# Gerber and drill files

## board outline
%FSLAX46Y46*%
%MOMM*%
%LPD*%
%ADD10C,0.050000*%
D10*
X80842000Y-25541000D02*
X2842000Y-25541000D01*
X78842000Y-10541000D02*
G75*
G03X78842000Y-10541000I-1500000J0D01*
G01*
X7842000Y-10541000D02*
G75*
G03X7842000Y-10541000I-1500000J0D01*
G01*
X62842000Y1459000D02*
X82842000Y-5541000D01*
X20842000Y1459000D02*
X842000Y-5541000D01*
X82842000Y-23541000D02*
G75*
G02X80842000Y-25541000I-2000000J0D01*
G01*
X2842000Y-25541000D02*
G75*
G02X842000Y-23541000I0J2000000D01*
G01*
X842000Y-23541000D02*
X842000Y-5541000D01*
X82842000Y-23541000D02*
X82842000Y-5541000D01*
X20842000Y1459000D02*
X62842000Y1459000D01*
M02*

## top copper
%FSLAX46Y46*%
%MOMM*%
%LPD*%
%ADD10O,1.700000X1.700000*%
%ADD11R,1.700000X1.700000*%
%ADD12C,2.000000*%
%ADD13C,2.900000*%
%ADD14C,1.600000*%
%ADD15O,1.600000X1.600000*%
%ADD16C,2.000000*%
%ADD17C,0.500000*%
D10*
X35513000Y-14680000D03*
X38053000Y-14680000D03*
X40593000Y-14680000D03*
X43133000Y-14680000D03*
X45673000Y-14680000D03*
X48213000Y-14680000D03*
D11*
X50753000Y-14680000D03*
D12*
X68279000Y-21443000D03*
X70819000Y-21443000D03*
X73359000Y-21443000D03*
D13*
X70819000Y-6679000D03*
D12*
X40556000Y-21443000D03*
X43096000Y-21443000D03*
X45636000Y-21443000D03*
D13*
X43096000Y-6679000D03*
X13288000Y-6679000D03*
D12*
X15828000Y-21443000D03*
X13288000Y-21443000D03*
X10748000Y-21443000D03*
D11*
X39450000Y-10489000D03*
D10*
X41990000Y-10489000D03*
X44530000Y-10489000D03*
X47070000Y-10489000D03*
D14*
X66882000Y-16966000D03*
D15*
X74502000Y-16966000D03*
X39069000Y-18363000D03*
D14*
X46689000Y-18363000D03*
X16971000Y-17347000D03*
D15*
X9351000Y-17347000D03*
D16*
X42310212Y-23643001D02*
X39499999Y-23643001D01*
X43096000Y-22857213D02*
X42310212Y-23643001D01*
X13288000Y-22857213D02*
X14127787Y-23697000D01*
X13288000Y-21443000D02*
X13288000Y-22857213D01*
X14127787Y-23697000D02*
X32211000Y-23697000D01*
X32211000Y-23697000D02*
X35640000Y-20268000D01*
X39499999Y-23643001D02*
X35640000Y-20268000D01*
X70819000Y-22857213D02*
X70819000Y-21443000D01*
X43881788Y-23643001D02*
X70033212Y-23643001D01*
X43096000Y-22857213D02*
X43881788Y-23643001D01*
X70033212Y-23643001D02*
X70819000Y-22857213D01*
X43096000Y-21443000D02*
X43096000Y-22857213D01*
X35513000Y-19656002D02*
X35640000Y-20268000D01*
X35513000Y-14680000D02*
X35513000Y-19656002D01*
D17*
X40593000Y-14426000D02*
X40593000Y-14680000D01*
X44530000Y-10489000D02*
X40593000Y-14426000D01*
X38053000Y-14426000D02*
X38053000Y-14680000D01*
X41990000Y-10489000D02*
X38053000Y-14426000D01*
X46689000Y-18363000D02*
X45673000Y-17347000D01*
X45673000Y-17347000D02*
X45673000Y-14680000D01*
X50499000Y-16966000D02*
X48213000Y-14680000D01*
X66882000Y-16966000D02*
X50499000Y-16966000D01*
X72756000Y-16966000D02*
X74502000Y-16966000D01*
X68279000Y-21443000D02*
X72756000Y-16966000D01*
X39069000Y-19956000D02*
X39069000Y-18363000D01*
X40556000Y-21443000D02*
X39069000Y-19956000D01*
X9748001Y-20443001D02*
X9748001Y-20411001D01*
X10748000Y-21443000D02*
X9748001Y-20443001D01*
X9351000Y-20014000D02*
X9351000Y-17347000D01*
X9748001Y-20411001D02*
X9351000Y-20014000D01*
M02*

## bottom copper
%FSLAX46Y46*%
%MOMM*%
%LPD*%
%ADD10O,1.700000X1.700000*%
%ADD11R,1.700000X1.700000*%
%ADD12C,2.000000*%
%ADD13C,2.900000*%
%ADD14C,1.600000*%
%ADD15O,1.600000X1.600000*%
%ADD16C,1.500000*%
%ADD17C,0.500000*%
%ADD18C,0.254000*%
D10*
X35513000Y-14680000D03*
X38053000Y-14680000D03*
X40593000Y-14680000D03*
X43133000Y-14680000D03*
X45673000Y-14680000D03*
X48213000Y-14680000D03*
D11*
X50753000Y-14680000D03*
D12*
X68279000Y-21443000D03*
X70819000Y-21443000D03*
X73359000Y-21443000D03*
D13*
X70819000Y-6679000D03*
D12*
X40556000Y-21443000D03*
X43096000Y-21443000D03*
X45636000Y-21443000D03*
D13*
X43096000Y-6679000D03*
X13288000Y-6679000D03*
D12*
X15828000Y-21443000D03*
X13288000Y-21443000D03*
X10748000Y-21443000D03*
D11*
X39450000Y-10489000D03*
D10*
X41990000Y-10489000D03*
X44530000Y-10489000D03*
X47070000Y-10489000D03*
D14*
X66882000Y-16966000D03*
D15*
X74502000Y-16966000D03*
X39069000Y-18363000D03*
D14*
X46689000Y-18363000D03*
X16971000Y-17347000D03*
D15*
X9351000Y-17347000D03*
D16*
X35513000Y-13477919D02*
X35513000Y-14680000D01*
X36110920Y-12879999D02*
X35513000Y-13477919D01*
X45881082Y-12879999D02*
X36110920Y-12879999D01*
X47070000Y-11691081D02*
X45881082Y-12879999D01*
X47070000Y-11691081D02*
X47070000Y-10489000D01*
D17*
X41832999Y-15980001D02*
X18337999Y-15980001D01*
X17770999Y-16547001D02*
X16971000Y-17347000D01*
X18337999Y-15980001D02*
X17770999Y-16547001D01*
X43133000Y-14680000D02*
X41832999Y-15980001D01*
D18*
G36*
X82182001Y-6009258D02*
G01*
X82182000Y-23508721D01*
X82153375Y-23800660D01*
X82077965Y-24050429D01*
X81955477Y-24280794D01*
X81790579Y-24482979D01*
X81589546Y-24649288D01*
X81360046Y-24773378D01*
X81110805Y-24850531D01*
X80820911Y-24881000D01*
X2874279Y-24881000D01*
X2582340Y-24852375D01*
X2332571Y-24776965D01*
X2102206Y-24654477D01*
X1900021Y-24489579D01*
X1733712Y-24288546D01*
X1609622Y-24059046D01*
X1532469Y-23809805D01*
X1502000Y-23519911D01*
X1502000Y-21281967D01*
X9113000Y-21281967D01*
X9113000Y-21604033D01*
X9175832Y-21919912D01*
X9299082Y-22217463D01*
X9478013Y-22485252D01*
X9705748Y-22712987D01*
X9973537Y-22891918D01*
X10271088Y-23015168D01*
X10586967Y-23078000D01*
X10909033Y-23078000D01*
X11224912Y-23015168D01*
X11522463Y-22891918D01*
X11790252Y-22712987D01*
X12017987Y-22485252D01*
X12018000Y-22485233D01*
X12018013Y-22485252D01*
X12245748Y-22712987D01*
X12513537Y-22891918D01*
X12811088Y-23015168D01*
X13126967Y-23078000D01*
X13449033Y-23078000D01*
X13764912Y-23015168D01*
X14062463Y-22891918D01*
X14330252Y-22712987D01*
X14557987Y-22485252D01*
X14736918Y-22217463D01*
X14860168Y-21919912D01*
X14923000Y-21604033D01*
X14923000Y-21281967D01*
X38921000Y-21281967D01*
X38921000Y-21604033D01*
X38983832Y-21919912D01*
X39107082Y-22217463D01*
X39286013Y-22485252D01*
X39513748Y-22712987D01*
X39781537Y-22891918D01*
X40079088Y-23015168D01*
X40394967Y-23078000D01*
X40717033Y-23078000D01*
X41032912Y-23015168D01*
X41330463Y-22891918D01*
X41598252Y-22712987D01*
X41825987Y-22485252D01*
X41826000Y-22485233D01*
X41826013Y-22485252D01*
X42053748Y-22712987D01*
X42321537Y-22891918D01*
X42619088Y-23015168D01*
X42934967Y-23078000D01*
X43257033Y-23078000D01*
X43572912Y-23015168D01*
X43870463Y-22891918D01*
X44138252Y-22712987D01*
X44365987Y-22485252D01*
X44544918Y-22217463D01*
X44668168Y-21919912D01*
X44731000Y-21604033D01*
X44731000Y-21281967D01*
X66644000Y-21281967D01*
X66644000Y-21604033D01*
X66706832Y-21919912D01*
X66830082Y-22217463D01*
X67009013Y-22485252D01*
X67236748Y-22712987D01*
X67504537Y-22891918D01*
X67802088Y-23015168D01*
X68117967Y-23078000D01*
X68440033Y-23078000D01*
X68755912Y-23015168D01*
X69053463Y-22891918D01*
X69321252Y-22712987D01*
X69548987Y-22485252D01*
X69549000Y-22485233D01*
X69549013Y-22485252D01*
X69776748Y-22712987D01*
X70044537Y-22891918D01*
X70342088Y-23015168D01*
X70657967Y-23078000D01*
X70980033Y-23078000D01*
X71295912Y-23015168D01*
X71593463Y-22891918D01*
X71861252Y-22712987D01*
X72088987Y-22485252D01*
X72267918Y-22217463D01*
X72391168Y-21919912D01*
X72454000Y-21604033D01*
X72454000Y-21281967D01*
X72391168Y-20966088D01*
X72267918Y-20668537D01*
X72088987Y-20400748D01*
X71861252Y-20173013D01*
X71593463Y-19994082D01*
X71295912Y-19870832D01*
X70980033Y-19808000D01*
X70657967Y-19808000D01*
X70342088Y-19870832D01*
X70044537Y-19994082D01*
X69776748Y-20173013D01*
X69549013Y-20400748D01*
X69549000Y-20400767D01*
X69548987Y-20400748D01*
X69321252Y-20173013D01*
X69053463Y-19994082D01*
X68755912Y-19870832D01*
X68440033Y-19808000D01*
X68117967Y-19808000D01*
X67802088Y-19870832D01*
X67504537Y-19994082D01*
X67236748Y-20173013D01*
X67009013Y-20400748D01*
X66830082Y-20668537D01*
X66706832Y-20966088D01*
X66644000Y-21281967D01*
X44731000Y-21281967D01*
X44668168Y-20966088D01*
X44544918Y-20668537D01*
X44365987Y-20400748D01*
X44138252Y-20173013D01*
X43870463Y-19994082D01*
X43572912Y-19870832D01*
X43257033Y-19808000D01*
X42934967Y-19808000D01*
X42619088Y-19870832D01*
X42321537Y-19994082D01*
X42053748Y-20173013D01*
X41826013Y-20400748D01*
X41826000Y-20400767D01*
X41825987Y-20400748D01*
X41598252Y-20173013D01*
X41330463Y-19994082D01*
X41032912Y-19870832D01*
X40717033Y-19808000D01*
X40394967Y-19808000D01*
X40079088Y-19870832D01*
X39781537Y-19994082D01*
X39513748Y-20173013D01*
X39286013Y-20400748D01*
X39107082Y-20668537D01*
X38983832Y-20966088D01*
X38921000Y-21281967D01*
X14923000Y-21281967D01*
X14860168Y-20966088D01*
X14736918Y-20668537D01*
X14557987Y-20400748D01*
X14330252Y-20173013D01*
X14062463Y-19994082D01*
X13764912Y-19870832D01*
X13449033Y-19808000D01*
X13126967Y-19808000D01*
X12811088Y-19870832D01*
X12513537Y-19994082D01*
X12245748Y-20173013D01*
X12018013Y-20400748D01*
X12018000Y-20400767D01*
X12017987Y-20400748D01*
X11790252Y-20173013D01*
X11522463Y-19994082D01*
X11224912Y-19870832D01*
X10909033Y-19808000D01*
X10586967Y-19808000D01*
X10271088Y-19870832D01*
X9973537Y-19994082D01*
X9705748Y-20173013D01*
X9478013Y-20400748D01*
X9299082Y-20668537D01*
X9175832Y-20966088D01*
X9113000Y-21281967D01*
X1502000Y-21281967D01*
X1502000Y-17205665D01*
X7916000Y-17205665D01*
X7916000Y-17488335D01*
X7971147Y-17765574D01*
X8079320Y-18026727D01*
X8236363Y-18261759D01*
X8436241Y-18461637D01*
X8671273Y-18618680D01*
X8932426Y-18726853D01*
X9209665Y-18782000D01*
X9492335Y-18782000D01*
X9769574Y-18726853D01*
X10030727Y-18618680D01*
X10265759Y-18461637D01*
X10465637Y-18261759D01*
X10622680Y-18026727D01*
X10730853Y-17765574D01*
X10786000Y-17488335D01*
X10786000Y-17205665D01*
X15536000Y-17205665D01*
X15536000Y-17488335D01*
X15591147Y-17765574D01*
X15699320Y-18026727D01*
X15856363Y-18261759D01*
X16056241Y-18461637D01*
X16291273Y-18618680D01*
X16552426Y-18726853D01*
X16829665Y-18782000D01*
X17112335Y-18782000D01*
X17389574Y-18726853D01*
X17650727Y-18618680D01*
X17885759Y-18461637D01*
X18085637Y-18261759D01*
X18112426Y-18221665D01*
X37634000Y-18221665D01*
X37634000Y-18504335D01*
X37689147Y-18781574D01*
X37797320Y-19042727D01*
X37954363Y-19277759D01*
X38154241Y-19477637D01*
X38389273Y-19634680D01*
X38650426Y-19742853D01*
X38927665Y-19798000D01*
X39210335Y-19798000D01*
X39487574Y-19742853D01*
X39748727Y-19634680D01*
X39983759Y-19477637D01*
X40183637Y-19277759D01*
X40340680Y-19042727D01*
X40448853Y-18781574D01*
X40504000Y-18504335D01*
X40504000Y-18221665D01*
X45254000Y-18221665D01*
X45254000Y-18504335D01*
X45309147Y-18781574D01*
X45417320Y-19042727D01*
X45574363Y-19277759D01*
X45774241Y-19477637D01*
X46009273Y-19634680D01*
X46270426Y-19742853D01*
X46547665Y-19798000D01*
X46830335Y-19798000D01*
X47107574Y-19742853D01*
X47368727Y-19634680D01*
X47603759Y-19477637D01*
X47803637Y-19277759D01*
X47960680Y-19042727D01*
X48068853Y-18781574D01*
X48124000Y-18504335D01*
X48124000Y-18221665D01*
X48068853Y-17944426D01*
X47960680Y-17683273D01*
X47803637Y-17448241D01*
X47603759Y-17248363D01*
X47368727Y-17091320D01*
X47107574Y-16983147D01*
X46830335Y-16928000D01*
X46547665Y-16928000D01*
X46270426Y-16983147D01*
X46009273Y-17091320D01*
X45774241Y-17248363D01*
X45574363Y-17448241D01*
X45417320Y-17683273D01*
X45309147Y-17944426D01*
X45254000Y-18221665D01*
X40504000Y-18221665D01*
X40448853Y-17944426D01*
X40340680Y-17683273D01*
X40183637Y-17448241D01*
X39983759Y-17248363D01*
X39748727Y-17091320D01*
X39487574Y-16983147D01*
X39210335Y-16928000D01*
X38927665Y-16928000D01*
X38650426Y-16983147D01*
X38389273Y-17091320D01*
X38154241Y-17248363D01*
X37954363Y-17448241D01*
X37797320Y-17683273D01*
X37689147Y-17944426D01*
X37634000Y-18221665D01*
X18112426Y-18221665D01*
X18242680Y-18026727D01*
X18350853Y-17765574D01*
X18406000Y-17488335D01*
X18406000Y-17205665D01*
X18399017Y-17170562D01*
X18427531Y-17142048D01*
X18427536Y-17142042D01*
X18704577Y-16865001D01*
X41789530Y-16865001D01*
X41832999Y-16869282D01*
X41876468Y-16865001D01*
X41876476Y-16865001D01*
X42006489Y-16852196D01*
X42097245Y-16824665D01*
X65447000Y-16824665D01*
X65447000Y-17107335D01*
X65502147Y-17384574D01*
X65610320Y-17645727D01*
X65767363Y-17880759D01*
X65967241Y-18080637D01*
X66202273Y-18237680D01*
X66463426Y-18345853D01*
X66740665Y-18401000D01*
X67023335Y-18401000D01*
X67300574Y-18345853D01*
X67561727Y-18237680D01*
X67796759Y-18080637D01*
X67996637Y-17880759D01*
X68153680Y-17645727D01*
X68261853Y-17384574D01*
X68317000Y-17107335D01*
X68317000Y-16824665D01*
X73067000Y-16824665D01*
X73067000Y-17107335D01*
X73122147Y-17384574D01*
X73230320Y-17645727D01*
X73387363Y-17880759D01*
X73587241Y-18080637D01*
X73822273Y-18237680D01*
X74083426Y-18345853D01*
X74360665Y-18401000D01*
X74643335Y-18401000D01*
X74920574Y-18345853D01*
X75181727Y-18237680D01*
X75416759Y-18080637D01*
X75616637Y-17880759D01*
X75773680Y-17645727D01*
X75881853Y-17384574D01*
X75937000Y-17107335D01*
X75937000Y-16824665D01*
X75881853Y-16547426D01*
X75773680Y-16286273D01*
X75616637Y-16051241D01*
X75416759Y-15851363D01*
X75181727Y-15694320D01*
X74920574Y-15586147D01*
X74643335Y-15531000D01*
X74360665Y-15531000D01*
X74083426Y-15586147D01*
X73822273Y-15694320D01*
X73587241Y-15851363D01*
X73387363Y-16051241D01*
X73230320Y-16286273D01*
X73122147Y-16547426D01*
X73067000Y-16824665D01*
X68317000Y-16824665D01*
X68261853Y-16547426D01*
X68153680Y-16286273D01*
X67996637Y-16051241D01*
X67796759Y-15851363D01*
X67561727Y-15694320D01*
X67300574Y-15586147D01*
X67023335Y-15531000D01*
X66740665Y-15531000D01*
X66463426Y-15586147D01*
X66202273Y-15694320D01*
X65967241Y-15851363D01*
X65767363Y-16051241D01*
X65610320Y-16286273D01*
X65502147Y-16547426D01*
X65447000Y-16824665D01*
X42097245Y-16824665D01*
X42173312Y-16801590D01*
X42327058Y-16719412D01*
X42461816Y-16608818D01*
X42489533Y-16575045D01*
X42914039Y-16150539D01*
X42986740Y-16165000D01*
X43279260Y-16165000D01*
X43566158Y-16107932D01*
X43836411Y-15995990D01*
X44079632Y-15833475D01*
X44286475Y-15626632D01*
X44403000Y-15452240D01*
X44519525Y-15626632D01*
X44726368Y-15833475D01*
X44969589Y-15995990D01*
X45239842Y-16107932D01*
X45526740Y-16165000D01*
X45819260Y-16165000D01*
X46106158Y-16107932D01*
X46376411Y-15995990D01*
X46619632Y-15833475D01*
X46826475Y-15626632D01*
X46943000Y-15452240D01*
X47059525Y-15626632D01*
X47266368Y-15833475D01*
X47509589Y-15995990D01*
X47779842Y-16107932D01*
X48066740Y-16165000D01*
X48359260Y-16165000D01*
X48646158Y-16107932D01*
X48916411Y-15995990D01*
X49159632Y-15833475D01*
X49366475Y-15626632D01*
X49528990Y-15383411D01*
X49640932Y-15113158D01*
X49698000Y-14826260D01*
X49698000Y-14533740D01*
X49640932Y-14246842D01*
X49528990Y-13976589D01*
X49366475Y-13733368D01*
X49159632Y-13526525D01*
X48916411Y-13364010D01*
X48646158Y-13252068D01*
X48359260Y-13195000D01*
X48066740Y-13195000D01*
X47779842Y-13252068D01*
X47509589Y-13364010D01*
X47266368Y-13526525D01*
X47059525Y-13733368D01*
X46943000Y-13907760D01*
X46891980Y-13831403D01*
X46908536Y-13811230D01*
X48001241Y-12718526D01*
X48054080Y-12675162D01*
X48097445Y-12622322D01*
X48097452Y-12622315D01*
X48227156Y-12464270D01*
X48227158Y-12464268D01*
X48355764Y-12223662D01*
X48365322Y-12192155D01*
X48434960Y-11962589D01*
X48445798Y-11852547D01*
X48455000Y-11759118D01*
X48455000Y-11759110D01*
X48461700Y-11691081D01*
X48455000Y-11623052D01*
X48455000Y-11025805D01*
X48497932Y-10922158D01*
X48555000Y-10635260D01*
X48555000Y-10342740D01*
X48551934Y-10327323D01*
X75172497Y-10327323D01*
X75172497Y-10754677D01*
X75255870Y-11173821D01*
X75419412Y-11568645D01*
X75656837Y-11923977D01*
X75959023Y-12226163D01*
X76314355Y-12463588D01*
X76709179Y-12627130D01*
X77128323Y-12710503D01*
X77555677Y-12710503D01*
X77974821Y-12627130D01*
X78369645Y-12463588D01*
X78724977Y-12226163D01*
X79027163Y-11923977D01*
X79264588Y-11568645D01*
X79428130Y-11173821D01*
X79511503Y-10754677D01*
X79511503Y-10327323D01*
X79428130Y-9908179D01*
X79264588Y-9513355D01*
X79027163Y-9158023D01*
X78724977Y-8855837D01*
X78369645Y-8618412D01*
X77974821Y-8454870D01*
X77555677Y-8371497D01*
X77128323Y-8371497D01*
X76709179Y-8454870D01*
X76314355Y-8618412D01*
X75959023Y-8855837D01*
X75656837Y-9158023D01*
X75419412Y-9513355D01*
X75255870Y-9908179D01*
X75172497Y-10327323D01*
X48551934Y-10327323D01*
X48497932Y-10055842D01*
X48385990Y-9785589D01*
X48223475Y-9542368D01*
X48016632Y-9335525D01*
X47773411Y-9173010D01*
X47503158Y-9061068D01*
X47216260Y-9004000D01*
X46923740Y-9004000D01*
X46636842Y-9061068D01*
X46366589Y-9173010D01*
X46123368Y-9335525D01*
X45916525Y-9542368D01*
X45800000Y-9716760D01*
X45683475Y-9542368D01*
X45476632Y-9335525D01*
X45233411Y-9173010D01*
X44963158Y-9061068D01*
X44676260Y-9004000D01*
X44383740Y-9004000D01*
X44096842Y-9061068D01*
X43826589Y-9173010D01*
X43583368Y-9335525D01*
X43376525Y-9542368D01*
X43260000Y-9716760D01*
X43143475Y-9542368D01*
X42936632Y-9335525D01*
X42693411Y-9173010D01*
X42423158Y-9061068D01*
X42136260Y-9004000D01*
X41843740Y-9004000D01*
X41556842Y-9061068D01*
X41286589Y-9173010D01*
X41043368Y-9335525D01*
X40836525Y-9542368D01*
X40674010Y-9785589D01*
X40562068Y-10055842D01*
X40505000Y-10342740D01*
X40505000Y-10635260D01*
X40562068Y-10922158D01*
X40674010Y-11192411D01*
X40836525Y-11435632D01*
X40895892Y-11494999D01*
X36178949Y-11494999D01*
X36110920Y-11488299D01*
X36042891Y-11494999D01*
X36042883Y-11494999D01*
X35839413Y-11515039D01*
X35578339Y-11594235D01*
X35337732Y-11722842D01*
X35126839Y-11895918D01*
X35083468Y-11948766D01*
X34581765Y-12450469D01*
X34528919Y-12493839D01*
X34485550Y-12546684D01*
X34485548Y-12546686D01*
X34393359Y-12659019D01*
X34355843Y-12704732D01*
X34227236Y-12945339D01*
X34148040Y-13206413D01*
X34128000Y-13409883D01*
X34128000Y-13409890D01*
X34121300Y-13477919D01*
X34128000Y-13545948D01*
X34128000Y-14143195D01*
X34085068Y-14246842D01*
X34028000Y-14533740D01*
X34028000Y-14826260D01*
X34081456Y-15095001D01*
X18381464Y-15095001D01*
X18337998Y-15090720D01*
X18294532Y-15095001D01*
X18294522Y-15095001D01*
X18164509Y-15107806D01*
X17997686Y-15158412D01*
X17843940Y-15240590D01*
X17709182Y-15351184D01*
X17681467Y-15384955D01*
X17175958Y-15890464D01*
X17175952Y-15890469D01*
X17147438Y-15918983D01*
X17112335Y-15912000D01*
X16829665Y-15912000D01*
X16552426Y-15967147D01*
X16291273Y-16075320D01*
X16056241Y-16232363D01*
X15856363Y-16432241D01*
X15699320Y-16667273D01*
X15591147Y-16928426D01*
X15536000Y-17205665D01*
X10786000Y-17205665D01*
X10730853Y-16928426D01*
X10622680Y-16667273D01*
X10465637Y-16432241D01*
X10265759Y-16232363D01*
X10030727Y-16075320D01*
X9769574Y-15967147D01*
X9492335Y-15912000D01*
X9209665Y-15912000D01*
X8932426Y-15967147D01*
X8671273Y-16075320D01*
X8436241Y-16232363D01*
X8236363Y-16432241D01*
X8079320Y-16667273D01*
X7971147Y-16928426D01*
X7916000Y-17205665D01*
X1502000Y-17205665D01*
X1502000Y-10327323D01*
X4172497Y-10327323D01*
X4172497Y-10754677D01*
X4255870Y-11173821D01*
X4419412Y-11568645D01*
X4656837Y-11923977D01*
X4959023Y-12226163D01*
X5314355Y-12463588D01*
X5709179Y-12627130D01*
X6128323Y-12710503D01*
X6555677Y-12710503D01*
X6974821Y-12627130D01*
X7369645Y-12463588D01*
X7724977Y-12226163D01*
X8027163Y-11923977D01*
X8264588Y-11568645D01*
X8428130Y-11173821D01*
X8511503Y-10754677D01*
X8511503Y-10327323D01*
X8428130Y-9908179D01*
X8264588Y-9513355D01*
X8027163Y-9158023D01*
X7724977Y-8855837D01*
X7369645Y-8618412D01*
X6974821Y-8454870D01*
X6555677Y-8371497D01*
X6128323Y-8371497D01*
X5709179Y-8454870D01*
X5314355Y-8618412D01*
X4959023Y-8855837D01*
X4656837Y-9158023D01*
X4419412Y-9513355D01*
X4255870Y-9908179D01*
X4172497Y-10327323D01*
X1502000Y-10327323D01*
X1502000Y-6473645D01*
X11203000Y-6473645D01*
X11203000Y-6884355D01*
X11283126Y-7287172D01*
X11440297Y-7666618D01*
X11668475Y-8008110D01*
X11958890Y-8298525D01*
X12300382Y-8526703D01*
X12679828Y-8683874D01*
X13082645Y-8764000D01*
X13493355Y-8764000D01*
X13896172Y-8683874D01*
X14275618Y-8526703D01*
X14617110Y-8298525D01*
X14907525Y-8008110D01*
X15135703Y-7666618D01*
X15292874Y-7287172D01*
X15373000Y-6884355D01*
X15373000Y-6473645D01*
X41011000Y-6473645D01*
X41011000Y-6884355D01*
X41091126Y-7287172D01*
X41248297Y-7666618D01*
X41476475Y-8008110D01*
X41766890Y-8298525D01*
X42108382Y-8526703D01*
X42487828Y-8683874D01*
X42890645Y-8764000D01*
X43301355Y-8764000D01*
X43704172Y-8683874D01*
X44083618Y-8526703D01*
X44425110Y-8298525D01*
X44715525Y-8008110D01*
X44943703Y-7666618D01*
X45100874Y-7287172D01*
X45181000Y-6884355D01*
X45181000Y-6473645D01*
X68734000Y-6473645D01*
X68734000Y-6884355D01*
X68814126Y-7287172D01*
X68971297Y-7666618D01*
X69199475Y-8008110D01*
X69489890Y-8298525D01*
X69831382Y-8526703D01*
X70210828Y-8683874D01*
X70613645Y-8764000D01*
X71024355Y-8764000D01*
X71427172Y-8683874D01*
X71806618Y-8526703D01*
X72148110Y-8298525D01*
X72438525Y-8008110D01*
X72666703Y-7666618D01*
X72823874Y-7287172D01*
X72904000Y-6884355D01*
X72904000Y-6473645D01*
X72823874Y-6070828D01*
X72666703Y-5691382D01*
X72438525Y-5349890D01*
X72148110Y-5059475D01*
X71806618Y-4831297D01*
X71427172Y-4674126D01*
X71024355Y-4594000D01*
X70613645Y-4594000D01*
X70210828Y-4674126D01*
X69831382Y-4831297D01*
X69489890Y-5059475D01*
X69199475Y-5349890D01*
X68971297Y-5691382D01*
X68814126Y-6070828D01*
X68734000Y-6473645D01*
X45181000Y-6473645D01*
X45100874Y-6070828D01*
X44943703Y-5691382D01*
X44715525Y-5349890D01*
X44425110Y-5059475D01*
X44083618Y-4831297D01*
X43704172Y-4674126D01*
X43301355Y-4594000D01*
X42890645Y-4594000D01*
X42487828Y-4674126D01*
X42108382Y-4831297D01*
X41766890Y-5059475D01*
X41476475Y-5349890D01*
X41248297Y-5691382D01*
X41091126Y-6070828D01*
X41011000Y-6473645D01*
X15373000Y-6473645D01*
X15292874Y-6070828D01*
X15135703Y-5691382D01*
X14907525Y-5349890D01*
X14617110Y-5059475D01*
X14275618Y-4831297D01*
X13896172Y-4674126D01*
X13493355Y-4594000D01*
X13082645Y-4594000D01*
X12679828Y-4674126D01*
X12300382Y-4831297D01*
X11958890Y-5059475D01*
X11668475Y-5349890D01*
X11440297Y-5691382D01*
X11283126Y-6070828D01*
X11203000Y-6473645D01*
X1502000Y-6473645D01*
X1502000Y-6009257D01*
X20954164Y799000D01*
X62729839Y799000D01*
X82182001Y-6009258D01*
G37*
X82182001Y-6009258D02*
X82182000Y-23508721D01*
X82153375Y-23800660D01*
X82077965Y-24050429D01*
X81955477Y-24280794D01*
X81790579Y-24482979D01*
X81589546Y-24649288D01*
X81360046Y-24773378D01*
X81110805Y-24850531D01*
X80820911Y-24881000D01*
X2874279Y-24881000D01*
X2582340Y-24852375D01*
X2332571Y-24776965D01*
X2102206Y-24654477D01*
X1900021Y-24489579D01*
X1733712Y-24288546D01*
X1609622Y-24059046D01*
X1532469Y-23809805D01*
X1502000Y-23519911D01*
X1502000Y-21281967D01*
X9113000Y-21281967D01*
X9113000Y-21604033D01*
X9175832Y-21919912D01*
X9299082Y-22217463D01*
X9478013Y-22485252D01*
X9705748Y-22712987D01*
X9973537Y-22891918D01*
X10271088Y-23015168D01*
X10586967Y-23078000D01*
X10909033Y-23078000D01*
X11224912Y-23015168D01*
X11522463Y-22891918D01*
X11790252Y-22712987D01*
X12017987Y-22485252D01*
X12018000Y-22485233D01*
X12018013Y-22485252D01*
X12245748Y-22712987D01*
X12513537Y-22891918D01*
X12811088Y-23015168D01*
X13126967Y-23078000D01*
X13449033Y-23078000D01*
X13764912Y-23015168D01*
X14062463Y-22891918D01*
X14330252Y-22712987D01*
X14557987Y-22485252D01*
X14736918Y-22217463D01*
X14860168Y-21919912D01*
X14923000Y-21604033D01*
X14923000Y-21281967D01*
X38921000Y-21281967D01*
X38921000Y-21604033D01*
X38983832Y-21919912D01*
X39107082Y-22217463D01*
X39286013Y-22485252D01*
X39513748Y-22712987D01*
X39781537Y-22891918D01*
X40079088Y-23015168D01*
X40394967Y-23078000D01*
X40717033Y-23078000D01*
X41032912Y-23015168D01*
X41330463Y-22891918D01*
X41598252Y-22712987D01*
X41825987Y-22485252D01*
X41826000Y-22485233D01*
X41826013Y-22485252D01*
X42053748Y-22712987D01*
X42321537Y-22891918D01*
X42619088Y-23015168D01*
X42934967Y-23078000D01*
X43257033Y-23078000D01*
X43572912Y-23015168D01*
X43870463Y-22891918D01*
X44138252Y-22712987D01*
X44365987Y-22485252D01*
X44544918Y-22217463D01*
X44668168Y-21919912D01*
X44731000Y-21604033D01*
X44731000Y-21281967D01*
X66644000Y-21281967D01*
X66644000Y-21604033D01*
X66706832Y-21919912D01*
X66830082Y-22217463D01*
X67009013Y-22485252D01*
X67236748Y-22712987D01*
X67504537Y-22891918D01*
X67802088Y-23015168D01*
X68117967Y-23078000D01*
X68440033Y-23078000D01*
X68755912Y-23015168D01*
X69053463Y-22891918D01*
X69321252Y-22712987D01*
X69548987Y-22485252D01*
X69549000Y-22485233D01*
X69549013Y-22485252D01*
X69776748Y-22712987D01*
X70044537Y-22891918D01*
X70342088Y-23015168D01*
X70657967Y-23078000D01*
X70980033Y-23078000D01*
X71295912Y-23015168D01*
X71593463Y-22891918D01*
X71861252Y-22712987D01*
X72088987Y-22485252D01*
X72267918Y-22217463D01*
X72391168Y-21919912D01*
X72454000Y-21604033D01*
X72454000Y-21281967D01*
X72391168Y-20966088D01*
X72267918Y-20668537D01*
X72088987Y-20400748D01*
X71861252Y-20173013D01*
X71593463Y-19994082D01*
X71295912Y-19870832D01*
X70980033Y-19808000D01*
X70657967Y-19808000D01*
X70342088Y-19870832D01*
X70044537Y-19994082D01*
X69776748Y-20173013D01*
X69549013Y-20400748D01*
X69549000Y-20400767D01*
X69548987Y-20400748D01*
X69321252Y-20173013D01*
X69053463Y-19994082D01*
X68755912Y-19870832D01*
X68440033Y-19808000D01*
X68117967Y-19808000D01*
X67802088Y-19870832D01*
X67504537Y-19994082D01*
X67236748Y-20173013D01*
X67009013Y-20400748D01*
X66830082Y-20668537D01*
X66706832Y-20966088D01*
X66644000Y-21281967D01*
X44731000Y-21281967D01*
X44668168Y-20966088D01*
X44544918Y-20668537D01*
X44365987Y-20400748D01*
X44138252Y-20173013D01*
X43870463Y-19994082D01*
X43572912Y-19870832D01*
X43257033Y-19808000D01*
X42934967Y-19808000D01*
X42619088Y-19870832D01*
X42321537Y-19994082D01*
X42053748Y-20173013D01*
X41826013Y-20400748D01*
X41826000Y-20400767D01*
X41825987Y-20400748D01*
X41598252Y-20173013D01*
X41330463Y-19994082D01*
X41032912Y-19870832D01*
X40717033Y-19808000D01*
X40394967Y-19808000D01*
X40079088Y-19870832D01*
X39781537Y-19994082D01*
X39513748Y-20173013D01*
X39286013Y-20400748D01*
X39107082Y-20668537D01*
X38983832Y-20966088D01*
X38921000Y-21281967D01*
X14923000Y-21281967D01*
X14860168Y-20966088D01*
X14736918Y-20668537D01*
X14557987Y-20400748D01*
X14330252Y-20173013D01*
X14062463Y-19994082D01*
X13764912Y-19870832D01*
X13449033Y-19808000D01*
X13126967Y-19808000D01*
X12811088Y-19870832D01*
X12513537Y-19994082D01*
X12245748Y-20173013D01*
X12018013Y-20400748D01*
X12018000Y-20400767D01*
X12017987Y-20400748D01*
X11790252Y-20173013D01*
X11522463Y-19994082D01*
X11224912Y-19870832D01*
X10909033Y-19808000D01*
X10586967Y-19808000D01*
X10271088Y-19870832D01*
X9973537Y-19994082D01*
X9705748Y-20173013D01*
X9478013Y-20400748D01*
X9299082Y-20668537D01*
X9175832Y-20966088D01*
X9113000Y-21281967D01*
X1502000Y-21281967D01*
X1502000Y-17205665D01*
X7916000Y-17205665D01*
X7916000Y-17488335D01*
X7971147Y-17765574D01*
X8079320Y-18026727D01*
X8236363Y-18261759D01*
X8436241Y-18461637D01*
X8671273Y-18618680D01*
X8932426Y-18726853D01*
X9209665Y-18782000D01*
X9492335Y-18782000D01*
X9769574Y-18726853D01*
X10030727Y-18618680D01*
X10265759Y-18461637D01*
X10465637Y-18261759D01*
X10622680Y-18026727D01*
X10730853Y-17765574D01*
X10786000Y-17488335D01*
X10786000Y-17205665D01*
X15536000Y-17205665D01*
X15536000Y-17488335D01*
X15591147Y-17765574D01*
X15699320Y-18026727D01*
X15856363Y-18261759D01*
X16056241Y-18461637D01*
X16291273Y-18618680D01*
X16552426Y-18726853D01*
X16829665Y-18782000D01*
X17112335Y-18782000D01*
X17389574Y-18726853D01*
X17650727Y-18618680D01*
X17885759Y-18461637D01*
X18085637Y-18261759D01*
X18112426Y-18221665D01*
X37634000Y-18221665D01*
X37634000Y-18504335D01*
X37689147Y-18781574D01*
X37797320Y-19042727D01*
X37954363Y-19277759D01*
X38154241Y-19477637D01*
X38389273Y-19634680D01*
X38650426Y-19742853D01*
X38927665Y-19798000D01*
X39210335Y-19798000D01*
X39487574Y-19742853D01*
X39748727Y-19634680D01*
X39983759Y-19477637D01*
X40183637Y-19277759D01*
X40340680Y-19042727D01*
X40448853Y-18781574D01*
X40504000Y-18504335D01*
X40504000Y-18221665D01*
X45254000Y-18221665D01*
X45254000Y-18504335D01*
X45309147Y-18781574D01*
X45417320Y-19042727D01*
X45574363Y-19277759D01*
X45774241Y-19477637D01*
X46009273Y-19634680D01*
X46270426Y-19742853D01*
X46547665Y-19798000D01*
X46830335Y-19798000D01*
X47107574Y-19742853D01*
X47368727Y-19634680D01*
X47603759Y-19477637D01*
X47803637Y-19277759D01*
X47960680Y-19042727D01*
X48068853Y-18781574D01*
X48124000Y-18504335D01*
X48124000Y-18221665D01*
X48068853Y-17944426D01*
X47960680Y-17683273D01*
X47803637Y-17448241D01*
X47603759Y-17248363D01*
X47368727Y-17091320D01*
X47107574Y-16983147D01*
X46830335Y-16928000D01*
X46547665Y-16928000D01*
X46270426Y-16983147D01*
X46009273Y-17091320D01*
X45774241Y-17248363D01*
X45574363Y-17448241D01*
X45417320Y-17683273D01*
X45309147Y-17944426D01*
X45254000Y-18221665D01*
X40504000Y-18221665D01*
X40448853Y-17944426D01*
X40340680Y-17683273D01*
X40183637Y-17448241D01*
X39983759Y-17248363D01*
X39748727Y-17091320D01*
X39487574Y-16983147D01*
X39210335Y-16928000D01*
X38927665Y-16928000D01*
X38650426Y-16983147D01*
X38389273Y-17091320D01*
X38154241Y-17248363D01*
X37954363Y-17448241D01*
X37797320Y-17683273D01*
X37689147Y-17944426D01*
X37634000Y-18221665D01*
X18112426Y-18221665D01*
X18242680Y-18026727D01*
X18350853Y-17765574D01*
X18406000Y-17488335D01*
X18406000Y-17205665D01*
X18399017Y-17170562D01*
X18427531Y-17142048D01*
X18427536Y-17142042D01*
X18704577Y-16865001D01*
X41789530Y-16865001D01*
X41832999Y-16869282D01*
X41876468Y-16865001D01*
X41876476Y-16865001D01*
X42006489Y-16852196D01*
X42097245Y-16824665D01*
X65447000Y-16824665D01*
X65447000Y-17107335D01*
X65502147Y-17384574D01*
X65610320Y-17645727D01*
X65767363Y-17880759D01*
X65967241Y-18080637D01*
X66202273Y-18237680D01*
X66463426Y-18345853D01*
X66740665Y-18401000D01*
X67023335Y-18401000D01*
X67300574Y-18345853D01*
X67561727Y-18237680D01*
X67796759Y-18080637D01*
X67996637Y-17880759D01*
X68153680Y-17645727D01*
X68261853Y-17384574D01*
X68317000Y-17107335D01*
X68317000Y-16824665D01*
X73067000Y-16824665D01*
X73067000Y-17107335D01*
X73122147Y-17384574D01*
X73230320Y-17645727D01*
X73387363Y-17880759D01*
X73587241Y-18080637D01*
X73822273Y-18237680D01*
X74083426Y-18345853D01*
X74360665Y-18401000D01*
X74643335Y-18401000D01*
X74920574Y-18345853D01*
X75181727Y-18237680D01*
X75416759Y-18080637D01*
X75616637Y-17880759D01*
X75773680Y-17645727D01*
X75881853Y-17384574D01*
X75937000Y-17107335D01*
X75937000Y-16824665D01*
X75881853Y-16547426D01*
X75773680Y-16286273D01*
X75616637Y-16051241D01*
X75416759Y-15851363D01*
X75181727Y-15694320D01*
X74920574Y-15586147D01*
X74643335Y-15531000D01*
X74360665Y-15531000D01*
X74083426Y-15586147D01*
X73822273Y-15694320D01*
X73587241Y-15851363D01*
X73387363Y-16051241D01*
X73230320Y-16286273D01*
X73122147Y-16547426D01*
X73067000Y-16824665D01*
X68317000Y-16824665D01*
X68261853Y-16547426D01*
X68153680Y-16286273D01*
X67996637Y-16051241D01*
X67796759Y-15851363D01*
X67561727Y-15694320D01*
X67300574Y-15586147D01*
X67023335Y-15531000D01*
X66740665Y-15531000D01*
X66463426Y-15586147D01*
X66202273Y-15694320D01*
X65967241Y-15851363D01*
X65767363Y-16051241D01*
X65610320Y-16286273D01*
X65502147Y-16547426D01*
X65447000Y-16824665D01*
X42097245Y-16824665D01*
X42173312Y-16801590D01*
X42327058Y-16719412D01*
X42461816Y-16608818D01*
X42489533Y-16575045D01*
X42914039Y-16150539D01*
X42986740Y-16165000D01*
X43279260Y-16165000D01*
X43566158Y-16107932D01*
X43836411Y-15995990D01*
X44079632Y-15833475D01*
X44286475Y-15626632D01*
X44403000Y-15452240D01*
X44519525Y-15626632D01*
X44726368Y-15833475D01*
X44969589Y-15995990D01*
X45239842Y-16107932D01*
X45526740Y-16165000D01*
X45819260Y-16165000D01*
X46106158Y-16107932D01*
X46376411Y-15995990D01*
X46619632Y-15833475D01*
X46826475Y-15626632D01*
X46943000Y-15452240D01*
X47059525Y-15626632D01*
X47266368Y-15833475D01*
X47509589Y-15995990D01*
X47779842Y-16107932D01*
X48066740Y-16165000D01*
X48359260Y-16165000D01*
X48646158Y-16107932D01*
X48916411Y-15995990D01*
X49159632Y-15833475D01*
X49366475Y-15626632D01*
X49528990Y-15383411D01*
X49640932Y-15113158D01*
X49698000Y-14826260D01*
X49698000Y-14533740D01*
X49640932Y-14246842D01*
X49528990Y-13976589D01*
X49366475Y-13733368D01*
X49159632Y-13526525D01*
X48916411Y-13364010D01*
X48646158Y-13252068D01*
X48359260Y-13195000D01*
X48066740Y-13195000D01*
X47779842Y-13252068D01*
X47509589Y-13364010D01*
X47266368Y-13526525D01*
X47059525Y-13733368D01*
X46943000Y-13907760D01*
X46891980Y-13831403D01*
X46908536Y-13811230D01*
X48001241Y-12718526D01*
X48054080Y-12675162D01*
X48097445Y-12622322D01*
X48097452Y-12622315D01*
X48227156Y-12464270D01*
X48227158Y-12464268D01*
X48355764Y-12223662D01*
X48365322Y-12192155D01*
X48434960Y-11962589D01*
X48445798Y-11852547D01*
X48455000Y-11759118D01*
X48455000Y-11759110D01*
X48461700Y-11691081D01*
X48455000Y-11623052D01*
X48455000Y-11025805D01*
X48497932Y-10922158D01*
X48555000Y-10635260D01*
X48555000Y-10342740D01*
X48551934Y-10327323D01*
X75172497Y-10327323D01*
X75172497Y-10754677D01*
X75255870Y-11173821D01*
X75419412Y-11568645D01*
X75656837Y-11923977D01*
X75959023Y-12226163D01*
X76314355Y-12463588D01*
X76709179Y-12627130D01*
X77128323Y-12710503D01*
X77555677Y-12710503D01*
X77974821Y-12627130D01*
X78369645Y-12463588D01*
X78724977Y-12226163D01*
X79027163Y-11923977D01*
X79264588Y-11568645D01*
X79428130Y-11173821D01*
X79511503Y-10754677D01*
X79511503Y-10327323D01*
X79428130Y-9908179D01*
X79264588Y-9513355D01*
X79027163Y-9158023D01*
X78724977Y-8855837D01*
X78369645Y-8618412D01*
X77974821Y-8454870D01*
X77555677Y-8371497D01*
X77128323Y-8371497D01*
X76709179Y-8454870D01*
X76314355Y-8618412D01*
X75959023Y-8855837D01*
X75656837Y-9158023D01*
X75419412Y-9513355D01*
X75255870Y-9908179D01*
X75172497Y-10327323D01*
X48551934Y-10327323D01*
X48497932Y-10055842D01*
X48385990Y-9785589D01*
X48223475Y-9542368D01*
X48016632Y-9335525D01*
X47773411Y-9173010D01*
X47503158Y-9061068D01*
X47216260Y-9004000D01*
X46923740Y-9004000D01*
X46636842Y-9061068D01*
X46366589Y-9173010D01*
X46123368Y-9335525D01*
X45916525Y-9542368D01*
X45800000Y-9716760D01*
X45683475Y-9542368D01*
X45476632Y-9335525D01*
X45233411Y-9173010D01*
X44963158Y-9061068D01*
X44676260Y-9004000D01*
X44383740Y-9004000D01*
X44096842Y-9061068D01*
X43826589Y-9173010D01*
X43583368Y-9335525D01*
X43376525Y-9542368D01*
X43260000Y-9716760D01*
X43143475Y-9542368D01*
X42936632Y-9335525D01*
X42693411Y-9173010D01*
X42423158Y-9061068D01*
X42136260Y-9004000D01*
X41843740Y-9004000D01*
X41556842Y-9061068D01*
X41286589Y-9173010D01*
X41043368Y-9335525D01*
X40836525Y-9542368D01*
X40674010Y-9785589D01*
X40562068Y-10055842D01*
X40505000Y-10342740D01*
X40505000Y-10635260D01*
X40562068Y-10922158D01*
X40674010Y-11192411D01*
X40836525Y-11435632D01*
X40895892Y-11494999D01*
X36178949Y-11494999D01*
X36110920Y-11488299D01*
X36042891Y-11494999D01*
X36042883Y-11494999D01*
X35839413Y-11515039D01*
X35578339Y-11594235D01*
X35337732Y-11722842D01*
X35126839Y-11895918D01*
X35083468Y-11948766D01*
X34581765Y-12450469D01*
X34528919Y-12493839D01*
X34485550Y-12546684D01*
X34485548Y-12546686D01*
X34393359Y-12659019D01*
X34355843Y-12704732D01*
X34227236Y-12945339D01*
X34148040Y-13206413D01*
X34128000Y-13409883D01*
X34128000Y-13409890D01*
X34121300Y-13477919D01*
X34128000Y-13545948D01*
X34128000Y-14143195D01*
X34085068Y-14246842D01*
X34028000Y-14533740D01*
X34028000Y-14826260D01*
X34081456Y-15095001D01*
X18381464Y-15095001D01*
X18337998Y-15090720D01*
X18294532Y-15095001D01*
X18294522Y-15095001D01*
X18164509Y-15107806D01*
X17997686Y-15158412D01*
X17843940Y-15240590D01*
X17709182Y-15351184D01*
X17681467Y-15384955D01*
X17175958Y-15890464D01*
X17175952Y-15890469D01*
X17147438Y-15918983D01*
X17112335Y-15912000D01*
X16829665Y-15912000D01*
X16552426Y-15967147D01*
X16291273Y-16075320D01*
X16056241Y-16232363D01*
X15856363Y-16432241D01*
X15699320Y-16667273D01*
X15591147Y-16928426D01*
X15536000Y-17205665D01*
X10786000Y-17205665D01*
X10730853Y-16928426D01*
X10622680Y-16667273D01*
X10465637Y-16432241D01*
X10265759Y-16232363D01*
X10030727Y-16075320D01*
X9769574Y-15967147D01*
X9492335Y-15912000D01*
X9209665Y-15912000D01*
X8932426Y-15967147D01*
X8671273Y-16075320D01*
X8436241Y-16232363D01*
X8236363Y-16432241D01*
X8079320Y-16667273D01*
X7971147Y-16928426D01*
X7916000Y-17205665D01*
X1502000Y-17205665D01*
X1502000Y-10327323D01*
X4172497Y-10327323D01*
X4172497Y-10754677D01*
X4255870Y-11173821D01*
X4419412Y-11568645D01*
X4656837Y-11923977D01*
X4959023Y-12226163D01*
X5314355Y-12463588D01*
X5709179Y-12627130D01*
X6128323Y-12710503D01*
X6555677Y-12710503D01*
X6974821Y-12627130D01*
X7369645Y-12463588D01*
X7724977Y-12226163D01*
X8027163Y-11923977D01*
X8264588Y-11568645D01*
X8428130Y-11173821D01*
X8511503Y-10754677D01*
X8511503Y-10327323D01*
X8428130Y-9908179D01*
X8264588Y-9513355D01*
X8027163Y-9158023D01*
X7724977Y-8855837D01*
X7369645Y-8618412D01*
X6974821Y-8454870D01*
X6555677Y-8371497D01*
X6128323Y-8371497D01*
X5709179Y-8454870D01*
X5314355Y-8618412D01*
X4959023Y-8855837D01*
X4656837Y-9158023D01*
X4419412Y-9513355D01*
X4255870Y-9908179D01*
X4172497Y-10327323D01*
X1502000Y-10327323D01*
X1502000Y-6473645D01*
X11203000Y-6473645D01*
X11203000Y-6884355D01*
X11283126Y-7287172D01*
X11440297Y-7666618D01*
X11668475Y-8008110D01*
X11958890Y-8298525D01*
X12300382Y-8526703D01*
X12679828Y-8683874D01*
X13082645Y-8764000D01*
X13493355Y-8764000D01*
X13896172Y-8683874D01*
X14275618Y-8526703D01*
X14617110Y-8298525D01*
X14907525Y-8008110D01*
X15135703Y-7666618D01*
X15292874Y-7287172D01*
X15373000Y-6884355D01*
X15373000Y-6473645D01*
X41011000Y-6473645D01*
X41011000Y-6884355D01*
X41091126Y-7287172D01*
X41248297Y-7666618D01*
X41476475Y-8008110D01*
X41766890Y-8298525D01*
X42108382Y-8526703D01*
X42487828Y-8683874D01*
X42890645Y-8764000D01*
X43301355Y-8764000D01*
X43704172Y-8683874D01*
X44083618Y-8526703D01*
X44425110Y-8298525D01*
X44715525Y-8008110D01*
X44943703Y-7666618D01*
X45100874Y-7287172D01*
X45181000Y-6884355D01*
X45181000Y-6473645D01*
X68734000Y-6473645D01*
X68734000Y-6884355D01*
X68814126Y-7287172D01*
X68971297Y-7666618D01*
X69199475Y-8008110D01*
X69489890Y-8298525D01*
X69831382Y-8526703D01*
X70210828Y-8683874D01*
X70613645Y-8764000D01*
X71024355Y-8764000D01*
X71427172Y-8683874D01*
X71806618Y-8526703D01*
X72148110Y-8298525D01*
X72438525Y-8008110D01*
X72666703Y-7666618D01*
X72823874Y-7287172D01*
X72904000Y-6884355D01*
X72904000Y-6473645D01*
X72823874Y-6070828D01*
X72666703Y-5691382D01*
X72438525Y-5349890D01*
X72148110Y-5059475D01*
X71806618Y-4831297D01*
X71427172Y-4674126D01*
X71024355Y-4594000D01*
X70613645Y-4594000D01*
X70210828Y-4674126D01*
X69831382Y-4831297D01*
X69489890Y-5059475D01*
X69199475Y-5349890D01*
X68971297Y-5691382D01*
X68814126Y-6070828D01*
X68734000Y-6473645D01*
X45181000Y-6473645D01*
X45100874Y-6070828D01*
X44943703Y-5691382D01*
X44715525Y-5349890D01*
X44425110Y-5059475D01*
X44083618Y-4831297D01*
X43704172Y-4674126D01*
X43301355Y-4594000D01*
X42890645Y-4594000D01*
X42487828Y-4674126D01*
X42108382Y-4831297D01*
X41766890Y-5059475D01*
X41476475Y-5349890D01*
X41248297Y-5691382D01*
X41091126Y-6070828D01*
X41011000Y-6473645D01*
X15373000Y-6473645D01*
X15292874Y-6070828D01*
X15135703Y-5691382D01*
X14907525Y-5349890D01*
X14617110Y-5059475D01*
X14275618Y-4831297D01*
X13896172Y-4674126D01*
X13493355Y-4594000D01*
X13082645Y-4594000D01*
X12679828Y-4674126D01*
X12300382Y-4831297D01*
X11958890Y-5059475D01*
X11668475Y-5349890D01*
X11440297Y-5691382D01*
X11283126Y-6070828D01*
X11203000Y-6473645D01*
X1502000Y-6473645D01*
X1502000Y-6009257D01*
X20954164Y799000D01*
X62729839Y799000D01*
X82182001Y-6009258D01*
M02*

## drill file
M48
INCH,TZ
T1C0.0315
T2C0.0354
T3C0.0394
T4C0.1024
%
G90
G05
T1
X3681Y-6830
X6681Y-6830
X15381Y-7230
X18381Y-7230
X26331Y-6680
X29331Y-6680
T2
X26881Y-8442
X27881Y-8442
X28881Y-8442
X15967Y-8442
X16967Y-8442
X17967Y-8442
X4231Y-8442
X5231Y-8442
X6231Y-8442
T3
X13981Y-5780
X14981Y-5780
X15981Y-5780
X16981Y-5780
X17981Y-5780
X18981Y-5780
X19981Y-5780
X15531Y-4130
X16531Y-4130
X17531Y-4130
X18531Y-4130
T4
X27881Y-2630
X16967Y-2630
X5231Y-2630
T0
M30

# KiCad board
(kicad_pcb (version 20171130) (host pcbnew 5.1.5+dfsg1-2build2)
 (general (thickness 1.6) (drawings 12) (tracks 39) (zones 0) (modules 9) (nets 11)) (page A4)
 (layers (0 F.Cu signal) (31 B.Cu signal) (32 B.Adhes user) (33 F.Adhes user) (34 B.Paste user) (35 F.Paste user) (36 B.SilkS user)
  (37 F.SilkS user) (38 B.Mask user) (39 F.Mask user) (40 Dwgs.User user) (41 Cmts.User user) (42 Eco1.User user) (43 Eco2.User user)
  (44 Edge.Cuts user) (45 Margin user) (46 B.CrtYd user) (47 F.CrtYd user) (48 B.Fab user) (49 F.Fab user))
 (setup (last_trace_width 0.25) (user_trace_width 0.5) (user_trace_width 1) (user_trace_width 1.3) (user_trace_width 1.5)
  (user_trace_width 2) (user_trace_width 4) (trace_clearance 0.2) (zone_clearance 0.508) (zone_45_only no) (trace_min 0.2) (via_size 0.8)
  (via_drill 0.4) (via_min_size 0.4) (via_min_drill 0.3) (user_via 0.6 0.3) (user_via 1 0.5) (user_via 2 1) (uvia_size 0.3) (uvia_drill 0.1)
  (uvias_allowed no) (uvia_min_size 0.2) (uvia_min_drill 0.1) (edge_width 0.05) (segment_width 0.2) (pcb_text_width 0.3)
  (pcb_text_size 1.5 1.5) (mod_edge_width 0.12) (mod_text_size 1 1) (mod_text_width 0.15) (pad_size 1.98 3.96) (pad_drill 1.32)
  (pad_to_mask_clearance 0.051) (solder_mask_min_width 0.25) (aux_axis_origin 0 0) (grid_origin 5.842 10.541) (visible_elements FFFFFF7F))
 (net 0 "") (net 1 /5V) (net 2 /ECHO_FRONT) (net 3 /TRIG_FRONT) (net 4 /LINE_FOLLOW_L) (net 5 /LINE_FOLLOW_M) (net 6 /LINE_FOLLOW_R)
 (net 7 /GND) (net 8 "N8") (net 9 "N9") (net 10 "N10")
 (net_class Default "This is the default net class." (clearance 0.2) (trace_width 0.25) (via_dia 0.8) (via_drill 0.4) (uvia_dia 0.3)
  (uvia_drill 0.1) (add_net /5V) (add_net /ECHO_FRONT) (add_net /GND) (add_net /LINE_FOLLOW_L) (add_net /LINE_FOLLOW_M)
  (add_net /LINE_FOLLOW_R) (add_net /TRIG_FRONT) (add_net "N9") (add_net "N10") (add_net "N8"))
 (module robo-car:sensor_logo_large (layer B.Cu) (at 57.531 12.065 180)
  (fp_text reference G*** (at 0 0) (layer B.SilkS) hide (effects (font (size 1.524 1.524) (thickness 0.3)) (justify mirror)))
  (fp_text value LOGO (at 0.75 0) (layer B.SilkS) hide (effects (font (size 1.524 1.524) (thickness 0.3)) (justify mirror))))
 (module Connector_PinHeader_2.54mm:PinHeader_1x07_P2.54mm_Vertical (layer F.Cu) (at 50.753 14.68 270)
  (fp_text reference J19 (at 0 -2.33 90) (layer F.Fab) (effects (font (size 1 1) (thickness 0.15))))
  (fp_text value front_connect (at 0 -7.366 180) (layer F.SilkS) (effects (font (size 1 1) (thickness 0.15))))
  (pad 7 thru_hole oval (at 0 15.24 270) (size 1.7 1.7) (drill 1) (layers *.Cu *.Mask) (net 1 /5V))
  (pad 6 thru_hole oval (at 0 12.7 270) (size 1.7 1.7) (drill 1) (layers *.Cu *.Mask) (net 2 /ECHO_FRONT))
  (pad 5 thru_hole oval (at 0 10.16 270) (size 1.7 1.7) (drill 1) (layers *.Cu *.Mask) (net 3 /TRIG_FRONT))
  (pad 4 thru_hole oval (at 0 7.62 270) (size 1.7 1.7) (drill 1) (layers *.Cu *.Mask) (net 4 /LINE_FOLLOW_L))
  (pad 3 thru_hole oval (at 0 5.08 270) (size 1.7 1.7) (drill 1) (layers *.Cu *.Mask) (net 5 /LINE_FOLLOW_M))
  (pad 2 thru_hole oval (at 0 2.54 270) (size 1.7 1.7) (drill 1) (layers *.Cu *.Mask) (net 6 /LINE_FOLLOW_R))
  (pad 1 thru_hole rect (at 0 0 270) (size 1.7 1.7) (drill 1) (layers *.Cu *.Mask) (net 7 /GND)))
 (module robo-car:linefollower (layer F.Cu) (at 70.565 6.933 90)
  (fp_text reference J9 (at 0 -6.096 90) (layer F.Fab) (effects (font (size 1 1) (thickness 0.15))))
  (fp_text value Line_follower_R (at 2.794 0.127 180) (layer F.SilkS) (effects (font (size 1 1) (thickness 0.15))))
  (pad 1 thru_hole circle (at -14.51 -2.286 90) (size 2 2) (drill 0.9) (layers *.Cu *.Mask) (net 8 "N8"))
  (pad 2 thru_hole circle (at -14.51 0.254 90) (size 2 2) (drill 0.9) (layers *.Cu *.Mask) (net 1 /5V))
  (pad 3 thru_hole circle (at -14.51 2.794 90) (size 2 2) (drill 0.9) (layers *.Cu *.Mask) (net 7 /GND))
  (pad 4 thru_hole circle (at 0.254 0.254 90) (size 2.9 2.9) (drill 2.6) (layers *.Cu *.Mask)))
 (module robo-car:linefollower (layer F.Cu) (at 42.842 6.933 90)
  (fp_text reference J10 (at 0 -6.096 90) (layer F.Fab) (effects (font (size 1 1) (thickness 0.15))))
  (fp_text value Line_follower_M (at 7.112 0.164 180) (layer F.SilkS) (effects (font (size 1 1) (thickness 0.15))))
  (pad 1 thru_hole circle (at -14.51 -2.286 90) (size 2 2) (drill 0.9) (layers *.Cu *.Mask) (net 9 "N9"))
  (pad 2 thru_hole circle (at -14.51 0.254 90) (size 2 2) (drill 0.9) (layers *.Cu *.Mask) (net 1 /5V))
  (pad 3 thru_hole circle (at -14.51 2.794 90) (size 2 2) (drill 0.9) (layers *.Cu *.Mask) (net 7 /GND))
  (pad 4 thru_hole circle (at 0.254 0.254 90) (size 2.9 2.9) (drill 2.6) (layers *.Cu *.Mask)))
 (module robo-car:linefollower (layer F.Cu) (at 13.034 6.933 90)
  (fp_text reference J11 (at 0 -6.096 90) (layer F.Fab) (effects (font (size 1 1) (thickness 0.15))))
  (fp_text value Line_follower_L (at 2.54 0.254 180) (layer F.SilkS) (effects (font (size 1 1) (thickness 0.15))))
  (pad 4 thru_hole circle (at 0.254 0.254 90) (size 2.9 2.9) (drill 2.6) (layers *.Cu *.Mask))
  (pad 3 thru_hole circle (at -14.51 2.794 90) (size 2 2) (drill 0.9) (layers *.Cu *.Mask) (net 7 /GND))
  (pad 2 thru_hole circle (at -14.51 0.254 90) (size 2 2) (drill 0.9) (layers *.Cu *.Mask) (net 1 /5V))
  (pad 1 thru_hole circle (at -14.51 -2.286 90) (size 2 2) (drill 0.9) (layers *.Cu *.Mask) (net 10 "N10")))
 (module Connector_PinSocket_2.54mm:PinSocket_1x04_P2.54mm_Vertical (layer F.Cu) (at 39.45 10.489 90)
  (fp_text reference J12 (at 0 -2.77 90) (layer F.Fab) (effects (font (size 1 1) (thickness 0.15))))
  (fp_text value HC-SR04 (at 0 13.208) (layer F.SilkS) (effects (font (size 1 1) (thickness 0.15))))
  (pad 1 thru_hole rect (at 0 0 90) (size 1.7 1.7) (drill 1) (layers *.Cu *.Mask) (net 7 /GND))
  (pad 2 thru_hole oval (at 0 2.54 90) (size 1.7 1.7) (drill 1) (layers *.Cu *.Mask) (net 2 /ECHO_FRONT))
  (pad 3 thru_hole oval (at 0 5.08 90) (size 1.7 1.7) (drill 1) (layers *.Cu *.Mask) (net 3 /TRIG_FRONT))
  (pad 4 thru_hole oval (at 0 7.62 90) (size 1.7 1.7) (drill 1) (layers *.Cu *.Mask) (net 1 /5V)))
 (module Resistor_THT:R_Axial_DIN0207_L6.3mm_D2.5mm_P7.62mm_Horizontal (layer F.Cu) (at 66.882 16.966)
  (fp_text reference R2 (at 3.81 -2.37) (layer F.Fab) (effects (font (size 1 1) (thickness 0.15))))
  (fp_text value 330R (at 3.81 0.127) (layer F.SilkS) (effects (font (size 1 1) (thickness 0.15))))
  (pad 1 thru_hole circle (at 0 0) (size 1.6 1.6) (drill 0.8) (layers *.Cu *.Mask) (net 6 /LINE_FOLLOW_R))
  (pad 2 thru_hole oval (at 7.62 0) (size 1.6 1.6) (drill 0.8) (layers *.Cu *.Mask) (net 8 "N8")))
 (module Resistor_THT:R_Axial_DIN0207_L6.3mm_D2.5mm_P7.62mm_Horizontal (layer F.Cu) (at 46.689 18.363 180)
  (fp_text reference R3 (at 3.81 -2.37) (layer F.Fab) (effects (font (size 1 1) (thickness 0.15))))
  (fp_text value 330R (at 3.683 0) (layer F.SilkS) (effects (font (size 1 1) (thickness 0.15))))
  (pad 2 thru_hole oval (at 7.62 0 180) (size 1.6 1.6) (drill 0.8) (layers *.Cu *.Mask) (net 9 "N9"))
  (pad 1 thru_hole circle (at 0 0 180) (size 1.6 1.6) (drill 0.8) (layers *.Cu *.Mask) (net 5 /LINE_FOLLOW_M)))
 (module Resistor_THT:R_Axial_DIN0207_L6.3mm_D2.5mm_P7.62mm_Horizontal (layer F.Cu) (at 16.971 17.347 180)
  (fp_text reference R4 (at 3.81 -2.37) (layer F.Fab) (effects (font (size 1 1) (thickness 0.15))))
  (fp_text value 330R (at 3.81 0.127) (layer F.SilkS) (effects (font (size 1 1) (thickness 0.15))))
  (pad 1 thru_hole circle (at 0 0 180) (size 1.6 1.6) (drill 0.8) (layers *.Cu *.Mask) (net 4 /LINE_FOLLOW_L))
  (pad 2 thru_hole oval (at 7.62 0 180) (size 1.6 1.6) (drill 0.8) (layers *.Cu *.Mask) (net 10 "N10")))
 (gr_line (start 80.842 25.541) (end 2.842 25.541) (layer Edge.Cuts) (width 0.05))
 (gr_circle (center 77.342 10.541) (end 78.842 10.541) (layer Edge.Cuts) (width 0.05))
 (gr_circle (center 6.342 10.541) (end 7.842 10.541) (layer Edge.Cuts) (width 0.05))
 (gr_line (start 62.842 -1.459) (end 82.842 5.541) (layer Edge.Cuts) (width 0.05))
 (gr_line (start 20.842 -1.459) (end 0.842 5.541) (layer Edge.Cuts) (width 0.05))
 (gr_arc (start 80.842 23.541) (end 80.842 25.541) (angle -90) (layer Edge.Cuts) (width 0.05))
 (gr_arc (start 2.842 23.541) (end 0.842 23.541) (angle -90) (layer Edge.Cuts) (width 0.05))
 (gr_line (start 0.842 23.541) (end 0.842 5.541) (layer Edge.Cuts) (width 0.05))
 (gr_line (start 82.842 23.541) (end 82.842 5.541) (layer Edge.Cuts) (width 0.05))
 (gr_line (start 20.842 -1.459) (end 62.842 -1.459) (layer Edge.Cuts) (width 0.05))
 (segment (start 42.310212 23.643001) (end 39.499999 23.643001) (width 2) (layer F.Cu) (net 1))
 (segment (start 43.096 22.857213) (end 42.310212 23.643001) (width 2) (layer F.Cu) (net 1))
 (segment (start 13.288 22.857213) (end 14.127787 23.697) (width 2) (layer F.Cu) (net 1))
 (segment (start 13.288 21.443) (end 13.288 22.857213) (width 2) (layer F.Cu) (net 1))
 (segment (start 14.127787 23.697) (end 32.211 23.697) (width 2) (layer F.Cu) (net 1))
 (segment (start 32.211 23.697) (end 35.64 20.268) (width 2) (layer F.Cu) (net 1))
 (segment (start 39.499999 23.643001) (end 35.64 20.268) (width 2) (layer F.Cu) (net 1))
 (segment (start 70.819 22.857213) (end 70.819 21.443) (width 2) (layer F.Cu) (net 1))
 (segment (start 43.881788 23.643001) (end 70.033212 23.643001) (width 2) (layer F.Cu) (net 1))
 (segment (start 43.096 22.857213) (end 43.881788 23.643001) (width 2) (layer F.Cu) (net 1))
 (segment (start 70.033212 23.643001) (end 70.819 22.857213) (width 2) (layer F.Cu) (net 1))
 (segment (start 43.096 21.443) (end 43.096 22.857213) (width 2) (layer F.Cu) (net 1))
 (segment (start 35.513 19.656002) (end 35.64 20.268) (width 2) (layer F.Cu) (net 1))
 (segment (start 35.513 14.68) (end 35.513 19.656002) (width 2) (layer F.Cu) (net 1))
 (segment (start 35.513 13.477919) (end 35.513 14.68) (width 1.5) (layer B.Cu) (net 1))
 (segment (start 36.11092 12.879999) (end 35.513 13.477919) (width 1.5) (layer B.Cu) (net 1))
 (segment (start 45.881082 12.879999) (end 36.11092 12.879999) (width 1.5) (layer B.Cu) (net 1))
 (segment (start 47.07 11.691081) (end 45.881082 12.879999) (width 1.5) (layer B.Cu) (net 1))
 (segment (start 47.07 11.691081) (end 47.07 10.489) (width 1.5) (layer B.Cu) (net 1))
 (segment (start 40.593 14.426) (end 40.593 14.68) (width 0.5) (layer F.Cu) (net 3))
 (segment (start 44.53 10.489) (end 40.593 14.426) (width 0.5) (layer F.Cu) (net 3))
 (segment (start 41.832999 15.980001) (end 18.337999 15.980001) (width 0.5) (layer B.Cu) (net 4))
 (segment (start 17.770999 16.547001) (end 16.971 17.347) (width 0.5) (layer B.Cu) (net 4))
 (segment (start 18.337999 15.980001) (end 17.770999 16.547001) (width 0.5) (layer B.Cu) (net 4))
 (segment (start 43.133 14.68) (end 41.832999 15.980001) (width 0.5) (layer B.Cu) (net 4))
 (segment (start 38.053 14.426) (end 38.053 14.68) (width 0.5) (layer F.Cu) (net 2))
 (segment (start 41.99 10.489) (end 38.053 14.426) (width 0.5) (layer F.Cu) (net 2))
 (segment (start 46.689 18.363) (end 45.673 17.347) (width 0.5) (layer F.Cu) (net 5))
 (segment (start 45.673 17.347) (end 45.673 14.68) (width 0.5) (layer F.Cu) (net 5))
 (segment (start 50.499 16.966) (end 48.213 14.68) (width 0.5) (layer F.Cu) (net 6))
 (segment (start 66.882 16.966) (end 50.499 16.966) (width 0.5) (layer F.Cu) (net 6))
 (segment (start 72.756 16.966) (end 74.502 16.966) (width 0.5) (layer F.Cu) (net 8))
 (segment (start 68.279 21.443) (end 72.756 16.966) (width 0.5) (layer F.Cu) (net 8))
 (segment (start 39.069 19.956) (end 39.069 18.363) (width 0.5) (layer F.Cu) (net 9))
 (segment (start 40.556 21.443) (end 39.069 19.956) (width 0.5) (layer F.Cu) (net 9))
 (segment (start 9.748001 20.443001) (end 9.748001 20.411001) (width 0.5) (layer F.Cu) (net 10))
 (segment (start 10.748 21.443) (end 9.748001 20.443001) (width 0.5) (layer F.Cu) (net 10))
 (segment (start 9.351 20.014) (end 9.351 17.347) (width 0.5) (layer F.Cu) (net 10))
 (segment (start 9.748001 20.411001) (end 9.351 20.014) (width 0.5) (layer F.Cu) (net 10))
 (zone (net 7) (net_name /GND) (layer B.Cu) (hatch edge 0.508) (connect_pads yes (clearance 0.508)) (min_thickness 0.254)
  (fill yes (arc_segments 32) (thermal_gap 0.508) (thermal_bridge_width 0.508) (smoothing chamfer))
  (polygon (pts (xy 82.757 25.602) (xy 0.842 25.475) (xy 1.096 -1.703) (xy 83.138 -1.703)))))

